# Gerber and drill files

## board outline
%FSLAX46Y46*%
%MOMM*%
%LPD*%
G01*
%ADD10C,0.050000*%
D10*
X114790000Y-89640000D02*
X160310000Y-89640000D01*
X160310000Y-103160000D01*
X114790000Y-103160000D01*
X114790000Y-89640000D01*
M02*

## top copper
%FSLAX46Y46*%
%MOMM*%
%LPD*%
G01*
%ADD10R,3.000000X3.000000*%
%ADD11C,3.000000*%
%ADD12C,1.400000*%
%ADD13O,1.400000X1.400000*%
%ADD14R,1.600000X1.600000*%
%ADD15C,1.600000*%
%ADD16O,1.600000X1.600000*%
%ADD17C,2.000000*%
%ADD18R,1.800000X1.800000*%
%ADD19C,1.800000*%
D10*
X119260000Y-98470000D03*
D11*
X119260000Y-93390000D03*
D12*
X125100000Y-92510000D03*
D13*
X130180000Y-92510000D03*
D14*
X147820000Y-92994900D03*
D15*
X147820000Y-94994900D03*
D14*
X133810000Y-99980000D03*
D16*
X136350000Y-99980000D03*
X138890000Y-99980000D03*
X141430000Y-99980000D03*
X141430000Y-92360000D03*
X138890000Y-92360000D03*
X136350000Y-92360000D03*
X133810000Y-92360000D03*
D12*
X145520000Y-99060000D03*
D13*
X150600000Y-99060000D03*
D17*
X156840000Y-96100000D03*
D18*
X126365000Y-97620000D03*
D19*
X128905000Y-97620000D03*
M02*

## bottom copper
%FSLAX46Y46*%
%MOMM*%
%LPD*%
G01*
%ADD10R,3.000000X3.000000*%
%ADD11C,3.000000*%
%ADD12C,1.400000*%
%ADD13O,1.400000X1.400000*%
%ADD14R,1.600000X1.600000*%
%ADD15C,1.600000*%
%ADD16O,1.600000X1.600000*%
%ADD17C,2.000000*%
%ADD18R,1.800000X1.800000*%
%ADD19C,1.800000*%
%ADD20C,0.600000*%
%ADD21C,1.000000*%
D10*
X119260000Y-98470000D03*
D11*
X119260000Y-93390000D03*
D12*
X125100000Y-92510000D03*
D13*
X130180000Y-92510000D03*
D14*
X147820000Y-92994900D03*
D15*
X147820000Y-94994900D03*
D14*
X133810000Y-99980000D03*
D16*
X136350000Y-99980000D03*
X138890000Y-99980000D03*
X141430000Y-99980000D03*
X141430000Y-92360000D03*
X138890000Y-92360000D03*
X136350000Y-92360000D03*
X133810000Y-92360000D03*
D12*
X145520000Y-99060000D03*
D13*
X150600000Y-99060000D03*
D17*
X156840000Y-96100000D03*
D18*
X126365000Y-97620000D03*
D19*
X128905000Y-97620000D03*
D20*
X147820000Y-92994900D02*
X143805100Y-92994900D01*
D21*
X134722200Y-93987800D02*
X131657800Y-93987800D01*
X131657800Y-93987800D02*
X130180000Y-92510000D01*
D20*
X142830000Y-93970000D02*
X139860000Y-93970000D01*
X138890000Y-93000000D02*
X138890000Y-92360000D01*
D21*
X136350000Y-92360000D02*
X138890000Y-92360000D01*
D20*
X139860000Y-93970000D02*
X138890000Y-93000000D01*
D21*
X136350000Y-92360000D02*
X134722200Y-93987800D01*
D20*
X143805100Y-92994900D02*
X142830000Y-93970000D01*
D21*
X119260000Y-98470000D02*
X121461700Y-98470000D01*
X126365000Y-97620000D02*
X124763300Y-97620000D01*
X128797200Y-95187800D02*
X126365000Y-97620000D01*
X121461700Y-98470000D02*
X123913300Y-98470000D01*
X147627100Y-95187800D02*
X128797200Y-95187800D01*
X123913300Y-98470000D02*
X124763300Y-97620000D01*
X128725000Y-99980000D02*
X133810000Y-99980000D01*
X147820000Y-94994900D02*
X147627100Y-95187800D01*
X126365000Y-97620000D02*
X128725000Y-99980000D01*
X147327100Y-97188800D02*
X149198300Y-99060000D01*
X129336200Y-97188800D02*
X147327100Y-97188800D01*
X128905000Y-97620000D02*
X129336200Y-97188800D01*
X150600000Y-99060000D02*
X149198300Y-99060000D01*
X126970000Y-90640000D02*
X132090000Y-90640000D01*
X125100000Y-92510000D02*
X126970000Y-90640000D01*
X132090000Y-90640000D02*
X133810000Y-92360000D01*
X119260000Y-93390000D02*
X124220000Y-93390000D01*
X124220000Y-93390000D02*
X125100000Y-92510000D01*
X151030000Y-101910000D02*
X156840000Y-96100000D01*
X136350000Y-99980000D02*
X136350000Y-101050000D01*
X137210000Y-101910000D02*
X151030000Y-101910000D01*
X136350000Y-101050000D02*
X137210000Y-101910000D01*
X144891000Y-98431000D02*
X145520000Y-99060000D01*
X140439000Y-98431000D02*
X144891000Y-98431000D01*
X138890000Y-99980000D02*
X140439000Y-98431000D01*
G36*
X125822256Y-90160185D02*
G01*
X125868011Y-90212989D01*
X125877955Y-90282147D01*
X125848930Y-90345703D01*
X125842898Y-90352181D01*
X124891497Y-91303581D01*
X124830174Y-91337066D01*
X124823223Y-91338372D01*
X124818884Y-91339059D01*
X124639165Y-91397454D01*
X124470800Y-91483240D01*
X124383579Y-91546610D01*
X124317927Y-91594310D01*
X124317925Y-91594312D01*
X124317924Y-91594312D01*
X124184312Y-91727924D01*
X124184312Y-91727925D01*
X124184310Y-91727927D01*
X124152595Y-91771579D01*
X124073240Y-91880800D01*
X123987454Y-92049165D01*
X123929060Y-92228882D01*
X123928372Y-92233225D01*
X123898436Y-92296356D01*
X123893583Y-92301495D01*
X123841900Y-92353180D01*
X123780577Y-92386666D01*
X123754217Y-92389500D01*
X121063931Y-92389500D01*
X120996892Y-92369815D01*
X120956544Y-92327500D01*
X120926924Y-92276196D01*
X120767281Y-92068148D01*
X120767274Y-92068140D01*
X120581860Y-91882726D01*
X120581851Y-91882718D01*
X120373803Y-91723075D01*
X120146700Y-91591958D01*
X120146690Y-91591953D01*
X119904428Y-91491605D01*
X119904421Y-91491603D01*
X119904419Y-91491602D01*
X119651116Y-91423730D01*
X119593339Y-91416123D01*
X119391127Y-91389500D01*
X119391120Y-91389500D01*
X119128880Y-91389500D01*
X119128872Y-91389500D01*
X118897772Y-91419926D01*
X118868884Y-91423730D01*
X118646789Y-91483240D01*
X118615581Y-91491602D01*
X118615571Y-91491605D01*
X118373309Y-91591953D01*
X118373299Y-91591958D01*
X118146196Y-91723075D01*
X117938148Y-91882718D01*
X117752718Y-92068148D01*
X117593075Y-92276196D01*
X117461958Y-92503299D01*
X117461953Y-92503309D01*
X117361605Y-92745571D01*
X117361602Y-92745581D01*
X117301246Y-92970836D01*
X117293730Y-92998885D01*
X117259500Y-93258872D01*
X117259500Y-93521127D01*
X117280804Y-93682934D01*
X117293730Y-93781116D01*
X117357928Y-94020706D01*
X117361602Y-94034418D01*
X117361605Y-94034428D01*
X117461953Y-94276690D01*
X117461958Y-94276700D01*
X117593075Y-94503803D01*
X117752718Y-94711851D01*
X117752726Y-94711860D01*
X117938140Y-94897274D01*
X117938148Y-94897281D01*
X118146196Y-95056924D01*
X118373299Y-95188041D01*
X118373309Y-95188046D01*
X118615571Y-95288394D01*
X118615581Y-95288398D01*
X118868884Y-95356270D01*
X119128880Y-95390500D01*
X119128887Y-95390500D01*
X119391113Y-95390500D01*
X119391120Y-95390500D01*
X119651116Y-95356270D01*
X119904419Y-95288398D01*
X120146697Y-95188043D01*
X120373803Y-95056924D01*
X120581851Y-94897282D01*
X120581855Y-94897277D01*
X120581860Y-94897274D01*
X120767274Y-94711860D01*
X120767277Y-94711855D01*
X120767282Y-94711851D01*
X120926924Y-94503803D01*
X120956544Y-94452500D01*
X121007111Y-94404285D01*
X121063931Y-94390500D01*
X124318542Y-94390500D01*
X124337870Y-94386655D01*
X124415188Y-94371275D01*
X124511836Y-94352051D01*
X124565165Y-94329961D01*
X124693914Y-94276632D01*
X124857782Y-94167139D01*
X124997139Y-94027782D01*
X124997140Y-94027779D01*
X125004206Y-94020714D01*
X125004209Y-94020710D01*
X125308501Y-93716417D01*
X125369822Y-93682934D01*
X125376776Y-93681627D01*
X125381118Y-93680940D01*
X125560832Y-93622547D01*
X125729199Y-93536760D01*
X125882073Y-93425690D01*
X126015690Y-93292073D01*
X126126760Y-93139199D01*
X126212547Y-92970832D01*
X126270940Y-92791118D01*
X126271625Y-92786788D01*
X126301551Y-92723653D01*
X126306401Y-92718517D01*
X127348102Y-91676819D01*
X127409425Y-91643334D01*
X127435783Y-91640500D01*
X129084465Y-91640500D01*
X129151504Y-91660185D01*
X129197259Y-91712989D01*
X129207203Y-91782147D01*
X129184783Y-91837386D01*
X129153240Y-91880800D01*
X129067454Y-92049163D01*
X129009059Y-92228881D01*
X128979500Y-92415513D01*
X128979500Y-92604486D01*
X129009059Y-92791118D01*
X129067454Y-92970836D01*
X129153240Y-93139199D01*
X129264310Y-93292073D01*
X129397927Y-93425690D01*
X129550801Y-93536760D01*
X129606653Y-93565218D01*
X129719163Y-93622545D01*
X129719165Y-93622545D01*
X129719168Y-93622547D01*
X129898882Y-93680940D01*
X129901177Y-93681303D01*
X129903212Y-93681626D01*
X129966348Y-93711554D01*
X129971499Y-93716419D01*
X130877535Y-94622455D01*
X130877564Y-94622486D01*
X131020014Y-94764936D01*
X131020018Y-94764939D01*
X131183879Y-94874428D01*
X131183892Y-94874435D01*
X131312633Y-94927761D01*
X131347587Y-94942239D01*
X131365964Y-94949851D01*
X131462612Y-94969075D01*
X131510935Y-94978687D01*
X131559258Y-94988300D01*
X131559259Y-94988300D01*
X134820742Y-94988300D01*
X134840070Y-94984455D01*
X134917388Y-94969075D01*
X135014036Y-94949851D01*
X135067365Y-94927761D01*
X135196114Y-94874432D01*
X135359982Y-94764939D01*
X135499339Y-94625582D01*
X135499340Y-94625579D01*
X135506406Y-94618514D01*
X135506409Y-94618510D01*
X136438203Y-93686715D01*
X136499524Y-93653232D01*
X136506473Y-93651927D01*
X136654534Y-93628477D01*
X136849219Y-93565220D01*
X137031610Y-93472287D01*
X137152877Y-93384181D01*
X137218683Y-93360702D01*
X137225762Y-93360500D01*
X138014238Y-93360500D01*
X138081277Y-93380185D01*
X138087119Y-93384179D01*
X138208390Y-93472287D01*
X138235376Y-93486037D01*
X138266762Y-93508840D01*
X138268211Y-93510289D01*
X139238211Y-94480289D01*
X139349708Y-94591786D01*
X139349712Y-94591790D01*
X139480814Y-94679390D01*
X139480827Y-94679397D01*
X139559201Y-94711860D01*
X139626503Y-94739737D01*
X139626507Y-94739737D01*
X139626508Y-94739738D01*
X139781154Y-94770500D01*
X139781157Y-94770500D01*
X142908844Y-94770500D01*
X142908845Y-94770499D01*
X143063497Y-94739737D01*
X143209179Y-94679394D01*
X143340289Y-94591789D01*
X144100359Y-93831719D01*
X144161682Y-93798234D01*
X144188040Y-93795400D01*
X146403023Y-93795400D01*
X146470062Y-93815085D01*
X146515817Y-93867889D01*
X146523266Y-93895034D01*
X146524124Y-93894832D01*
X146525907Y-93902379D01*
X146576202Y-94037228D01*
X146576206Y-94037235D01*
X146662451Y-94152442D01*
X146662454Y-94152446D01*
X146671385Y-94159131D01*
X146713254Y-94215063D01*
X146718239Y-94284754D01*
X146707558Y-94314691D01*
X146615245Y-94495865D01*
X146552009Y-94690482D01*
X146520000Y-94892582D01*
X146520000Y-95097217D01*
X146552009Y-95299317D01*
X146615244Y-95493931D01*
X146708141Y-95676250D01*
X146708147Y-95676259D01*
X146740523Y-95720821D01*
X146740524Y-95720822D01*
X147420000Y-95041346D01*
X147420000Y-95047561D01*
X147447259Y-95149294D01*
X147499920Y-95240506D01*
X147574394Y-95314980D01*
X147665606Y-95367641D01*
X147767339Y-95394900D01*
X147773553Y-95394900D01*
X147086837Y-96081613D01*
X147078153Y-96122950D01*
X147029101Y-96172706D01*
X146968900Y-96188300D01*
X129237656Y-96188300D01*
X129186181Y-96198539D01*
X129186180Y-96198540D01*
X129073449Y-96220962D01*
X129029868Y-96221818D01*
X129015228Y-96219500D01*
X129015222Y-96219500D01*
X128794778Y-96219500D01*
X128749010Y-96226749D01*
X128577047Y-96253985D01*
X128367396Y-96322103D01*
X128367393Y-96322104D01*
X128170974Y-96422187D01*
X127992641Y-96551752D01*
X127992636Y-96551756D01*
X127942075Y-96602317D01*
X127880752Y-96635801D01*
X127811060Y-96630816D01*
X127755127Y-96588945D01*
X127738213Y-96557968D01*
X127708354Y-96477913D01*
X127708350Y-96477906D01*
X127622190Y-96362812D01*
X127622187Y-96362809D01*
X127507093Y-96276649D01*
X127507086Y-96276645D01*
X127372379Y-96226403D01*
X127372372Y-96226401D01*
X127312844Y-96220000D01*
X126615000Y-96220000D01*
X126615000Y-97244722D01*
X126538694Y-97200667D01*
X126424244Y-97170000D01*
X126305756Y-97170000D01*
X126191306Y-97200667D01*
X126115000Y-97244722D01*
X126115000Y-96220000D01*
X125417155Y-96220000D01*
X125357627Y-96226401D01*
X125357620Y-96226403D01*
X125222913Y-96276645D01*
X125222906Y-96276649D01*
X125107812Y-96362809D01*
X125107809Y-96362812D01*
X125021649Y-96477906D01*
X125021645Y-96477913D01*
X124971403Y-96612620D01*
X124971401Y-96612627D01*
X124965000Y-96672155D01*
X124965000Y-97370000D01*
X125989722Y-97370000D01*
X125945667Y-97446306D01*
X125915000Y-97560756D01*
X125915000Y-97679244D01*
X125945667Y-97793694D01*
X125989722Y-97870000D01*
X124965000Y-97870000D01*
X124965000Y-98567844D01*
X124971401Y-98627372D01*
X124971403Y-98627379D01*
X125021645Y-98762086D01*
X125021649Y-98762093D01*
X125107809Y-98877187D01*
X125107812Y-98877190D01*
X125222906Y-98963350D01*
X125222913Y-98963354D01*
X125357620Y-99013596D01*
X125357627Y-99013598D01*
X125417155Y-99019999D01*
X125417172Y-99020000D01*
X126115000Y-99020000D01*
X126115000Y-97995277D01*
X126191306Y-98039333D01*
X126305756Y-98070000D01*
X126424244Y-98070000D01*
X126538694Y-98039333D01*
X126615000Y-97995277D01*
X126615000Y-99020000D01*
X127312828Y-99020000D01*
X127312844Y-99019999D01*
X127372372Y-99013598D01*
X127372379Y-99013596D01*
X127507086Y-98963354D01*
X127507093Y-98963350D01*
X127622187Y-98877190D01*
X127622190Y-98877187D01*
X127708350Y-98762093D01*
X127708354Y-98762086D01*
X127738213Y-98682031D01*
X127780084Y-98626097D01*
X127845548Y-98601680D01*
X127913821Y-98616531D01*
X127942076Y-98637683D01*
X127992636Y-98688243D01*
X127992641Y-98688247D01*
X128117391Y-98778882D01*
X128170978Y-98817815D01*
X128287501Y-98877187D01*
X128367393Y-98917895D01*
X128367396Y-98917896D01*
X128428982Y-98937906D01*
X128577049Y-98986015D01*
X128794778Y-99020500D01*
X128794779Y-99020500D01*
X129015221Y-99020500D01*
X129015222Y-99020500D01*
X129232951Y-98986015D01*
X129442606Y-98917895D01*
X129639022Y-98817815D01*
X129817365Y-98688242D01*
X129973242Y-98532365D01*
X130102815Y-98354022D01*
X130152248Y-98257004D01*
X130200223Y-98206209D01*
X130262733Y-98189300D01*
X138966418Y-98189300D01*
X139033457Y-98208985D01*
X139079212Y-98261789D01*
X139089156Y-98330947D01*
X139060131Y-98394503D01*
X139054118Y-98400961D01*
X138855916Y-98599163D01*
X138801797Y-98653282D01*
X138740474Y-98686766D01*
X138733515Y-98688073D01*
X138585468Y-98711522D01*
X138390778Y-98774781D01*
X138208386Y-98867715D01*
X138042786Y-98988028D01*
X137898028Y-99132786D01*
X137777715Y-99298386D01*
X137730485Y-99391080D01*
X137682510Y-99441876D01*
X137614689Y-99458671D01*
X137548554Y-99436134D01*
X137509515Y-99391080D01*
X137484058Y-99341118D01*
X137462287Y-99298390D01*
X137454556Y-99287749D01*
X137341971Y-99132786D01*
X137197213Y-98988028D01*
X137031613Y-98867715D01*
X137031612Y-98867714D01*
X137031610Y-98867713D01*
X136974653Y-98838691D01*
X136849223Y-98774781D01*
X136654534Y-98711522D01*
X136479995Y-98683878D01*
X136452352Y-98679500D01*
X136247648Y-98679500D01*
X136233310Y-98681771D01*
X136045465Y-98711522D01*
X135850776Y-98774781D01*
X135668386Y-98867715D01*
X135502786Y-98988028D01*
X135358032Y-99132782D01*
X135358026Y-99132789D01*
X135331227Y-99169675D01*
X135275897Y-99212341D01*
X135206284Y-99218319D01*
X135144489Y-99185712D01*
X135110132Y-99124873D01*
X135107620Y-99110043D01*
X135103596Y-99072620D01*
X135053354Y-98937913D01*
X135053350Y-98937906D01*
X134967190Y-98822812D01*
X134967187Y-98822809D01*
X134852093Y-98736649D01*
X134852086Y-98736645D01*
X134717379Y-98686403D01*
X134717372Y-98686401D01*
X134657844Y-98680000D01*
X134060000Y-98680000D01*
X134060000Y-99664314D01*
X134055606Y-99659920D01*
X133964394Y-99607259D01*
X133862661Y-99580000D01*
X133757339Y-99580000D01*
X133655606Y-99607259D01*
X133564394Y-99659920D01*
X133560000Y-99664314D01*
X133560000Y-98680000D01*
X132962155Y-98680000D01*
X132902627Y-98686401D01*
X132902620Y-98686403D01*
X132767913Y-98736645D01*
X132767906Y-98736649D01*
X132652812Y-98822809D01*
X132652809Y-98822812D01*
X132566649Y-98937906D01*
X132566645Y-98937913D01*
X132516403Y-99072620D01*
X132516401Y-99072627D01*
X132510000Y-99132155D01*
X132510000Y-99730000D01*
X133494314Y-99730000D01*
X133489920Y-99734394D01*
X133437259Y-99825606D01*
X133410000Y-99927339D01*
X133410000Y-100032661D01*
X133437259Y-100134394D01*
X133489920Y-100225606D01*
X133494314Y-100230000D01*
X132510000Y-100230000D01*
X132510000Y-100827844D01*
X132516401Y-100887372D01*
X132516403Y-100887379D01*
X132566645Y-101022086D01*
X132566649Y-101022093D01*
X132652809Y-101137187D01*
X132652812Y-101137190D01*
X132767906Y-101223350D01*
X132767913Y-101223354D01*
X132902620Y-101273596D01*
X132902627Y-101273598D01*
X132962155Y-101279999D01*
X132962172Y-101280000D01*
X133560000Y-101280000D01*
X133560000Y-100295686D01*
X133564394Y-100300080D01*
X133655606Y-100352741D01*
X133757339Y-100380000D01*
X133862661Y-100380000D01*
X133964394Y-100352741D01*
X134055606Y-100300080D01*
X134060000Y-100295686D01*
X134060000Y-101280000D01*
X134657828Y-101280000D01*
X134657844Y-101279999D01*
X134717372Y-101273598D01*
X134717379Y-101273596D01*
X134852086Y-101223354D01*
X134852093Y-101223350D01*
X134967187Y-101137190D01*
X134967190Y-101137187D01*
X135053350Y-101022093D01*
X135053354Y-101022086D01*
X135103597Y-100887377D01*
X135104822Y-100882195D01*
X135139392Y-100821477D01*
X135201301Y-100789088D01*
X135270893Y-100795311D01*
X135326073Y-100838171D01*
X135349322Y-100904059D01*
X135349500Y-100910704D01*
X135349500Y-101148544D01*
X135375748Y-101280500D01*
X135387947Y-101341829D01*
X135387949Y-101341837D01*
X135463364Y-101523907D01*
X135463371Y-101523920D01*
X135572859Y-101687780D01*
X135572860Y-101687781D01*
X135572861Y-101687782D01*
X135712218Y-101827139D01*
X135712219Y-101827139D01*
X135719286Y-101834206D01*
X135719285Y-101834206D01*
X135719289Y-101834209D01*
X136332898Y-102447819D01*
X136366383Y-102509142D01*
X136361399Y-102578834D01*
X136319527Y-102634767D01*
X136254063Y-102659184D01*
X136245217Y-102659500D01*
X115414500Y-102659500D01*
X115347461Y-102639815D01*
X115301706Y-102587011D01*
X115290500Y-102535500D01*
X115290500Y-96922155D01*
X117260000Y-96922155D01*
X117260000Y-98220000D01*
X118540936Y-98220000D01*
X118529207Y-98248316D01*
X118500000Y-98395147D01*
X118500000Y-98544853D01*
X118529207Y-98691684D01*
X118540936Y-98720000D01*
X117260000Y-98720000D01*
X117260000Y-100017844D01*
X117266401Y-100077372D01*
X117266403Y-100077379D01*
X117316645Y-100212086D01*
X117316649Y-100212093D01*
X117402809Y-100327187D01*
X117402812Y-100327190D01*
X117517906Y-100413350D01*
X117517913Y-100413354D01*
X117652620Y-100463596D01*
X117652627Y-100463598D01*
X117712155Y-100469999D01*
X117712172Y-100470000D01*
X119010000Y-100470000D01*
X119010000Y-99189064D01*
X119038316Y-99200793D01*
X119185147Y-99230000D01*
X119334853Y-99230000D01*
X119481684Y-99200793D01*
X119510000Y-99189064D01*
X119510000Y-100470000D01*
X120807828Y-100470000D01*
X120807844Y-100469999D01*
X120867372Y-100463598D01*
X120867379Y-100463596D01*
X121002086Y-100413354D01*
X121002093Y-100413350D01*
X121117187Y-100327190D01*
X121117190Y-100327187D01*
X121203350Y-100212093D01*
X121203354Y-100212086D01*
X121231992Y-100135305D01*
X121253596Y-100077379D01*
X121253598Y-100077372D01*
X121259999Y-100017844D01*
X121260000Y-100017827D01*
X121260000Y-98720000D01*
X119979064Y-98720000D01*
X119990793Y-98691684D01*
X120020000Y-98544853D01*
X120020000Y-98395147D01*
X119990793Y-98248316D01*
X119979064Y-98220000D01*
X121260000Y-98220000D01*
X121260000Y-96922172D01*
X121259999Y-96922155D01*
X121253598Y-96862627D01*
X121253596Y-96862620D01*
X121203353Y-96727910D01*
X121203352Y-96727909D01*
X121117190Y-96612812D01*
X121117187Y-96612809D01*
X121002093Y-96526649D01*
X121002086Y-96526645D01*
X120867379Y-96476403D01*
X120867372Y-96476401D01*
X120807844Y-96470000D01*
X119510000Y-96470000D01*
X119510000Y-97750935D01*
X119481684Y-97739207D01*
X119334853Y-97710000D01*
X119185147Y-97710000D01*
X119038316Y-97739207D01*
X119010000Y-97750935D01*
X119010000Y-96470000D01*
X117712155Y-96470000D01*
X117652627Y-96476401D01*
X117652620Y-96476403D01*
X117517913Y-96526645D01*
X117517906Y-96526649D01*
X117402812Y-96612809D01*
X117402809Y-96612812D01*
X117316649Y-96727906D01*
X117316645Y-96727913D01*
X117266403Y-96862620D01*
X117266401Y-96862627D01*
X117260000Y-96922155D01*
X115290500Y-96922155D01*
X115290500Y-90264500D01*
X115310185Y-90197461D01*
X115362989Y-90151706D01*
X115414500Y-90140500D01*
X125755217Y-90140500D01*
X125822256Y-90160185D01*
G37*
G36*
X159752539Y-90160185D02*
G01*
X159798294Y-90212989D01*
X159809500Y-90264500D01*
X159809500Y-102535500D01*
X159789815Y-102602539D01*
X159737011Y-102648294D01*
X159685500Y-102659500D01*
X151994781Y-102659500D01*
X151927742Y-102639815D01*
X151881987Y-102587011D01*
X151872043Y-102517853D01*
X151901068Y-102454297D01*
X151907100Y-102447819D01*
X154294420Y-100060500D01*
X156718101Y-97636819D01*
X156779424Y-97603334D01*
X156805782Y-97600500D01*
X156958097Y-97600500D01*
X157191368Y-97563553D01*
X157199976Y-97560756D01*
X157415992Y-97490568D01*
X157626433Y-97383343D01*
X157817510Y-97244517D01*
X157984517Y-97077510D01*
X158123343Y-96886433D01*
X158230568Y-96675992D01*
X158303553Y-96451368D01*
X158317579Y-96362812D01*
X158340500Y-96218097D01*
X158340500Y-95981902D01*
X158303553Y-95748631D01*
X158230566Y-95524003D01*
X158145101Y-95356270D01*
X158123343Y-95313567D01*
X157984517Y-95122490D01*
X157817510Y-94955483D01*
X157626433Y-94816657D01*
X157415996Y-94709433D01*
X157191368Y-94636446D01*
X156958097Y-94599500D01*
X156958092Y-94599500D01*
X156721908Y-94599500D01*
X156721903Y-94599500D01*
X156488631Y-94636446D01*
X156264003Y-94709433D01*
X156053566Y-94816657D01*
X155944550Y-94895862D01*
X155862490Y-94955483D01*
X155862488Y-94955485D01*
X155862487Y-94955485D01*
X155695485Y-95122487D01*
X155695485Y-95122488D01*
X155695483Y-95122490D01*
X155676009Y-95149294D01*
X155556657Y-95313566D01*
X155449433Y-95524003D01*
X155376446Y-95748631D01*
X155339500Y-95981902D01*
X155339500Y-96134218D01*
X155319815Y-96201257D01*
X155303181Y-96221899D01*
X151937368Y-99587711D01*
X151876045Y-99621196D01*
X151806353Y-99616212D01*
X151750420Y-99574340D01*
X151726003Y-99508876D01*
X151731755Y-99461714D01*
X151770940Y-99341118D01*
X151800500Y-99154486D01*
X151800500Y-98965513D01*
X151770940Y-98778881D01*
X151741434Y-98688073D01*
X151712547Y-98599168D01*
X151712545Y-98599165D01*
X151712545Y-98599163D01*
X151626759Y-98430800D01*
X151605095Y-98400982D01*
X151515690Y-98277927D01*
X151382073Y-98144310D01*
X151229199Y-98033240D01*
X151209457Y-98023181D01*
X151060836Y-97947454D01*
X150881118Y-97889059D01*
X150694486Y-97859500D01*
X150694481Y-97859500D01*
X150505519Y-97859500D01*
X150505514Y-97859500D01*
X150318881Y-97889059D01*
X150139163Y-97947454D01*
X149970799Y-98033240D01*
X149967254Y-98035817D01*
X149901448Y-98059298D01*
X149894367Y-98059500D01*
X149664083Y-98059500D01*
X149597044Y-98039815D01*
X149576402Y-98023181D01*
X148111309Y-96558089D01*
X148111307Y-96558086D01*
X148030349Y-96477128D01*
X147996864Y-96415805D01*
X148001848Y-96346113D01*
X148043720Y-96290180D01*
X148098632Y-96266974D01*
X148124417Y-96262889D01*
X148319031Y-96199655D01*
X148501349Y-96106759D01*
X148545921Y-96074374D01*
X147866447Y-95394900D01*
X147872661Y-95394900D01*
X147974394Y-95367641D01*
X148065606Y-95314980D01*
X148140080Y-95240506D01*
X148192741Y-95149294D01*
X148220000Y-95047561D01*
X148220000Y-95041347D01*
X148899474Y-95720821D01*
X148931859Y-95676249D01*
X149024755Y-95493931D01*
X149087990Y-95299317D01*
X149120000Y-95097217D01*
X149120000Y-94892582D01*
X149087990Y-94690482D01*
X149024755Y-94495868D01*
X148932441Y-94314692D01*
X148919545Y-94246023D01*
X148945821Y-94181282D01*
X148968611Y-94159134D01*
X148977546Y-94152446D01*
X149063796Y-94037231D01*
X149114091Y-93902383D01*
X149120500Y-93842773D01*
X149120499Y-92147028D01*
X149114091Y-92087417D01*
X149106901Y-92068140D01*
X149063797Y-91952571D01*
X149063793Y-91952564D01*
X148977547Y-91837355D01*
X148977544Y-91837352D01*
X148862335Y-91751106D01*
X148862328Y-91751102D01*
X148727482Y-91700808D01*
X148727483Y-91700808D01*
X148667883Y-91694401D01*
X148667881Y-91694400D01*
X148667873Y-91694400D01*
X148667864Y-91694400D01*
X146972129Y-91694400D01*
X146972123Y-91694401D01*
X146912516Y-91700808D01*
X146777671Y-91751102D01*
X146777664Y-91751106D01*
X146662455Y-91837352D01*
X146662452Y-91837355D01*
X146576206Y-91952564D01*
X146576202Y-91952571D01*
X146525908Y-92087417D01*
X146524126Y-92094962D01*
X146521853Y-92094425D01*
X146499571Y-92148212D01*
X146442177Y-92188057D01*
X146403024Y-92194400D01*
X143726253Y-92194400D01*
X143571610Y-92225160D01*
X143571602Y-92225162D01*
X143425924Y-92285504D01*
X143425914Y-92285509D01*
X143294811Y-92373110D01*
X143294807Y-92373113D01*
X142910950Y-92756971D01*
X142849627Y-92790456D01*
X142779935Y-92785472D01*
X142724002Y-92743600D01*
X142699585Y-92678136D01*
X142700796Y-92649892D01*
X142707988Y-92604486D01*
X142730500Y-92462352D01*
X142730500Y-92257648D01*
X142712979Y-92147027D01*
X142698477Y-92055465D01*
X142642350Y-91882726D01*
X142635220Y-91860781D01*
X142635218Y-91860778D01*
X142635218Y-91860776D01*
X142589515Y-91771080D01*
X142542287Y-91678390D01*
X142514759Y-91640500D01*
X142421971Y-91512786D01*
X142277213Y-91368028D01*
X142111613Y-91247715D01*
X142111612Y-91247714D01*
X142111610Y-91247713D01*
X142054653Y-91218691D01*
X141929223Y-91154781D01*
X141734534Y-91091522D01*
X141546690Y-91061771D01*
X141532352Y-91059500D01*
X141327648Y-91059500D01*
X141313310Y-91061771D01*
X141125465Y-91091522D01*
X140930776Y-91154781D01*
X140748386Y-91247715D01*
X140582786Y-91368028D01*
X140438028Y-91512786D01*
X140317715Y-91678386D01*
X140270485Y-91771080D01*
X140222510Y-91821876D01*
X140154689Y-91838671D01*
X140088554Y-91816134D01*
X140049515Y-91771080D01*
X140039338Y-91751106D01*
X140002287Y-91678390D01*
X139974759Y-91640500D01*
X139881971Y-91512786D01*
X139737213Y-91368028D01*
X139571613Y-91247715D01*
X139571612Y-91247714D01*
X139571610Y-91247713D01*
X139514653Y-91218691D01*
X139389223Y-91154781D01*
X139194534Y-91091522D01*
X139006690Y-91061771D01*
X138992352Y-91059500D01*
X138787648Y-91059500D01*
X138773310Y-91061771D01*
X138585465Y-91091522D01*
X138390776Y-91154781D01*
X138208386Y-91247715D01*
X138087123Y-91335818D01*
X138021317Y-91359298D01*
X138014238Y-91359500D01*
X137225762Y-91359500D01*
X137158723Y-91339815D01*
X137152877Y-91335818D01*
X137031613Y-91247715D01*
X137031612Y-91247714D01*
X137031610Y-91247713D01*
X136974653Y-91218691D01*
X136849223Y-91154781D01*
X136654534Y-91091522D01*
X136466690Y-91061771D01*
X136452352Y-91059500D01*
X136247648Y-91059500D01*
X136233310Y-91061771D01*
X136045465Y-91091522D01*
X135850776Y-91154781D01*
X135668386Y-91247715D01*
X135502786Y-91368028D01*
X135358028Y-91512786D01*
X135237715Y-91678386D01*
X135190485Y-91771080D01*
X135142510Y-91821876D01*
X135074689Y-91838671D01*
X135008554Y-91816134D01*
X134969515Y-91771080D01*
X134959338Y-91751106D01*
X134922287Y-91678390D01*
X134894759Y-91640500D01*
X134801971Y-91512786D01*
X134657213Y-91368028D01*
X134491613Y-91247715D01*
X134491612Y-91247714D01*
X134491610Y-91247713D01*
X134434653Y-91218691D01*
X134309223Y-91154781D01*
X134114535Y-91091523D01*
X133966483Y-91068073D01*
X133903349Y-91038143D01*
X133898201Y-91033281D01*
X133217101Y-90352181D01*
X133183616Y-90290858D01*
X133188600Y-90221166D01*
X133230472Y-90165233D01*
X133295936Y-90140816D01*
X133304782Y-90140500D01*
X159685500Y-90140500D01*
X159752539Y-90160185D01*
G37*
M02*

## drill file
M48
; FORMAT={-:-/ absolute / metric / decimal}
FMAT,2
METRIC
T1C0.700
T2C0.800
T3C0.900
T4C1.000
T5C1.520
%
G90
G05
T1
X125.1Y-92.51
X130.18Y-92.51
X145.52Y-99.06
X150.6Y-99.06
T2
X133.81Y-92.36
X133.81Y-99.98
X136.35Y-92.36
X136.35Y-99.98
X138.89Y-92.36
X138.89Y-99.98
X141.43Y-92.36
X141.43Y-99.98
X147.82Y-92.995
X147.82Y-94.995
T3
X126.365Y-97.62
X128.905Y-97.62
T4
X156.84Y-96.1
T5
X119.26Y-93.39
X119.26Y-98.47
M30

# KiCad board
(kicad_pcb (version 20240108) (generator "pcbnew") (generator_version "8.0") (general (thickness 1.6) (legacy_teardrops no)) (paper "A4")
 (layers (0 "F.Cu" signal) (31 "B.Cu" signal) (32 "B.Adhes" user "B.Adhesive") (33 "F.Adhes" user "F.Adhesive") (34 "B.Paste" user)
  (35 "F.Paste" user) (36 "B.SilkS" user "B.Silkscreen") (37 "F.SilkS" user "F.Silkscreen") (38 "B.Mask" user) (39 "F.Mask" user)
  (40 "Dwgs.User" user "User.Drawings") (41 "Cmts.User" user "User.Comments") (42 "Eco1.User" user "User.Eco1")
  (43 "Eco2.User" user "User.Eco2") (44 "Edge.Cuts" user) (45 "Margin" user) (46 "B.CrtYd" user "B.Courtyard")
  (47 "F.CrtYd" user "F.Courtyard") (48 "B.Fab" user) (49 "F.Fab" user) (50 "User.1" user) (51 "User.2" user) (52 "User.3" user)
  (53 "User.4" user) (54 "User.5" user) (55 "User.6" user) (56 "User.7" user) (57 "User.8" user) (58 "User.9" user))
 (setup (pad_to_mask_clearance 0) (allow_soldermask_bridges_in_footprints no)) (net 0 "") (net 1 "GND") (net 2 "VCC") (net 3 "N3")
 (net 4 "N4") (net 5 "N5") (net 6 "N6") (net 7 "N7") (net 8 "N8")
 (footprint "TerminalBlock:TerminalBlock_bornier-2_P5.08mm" (layer "F.Cu") (at 119.26 98.47 90)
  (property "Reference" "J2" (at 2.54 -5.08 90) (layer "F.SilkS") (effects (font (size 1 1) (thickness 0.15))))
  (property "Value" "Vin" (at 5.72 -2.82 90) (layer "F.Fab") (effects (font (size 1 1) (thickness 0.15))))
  (pad "1" thru_hole rect (at 0 0 90) (size 3 3) (drill 1.52) (layers "*.Cu" "*.Mask") (remove_unused_layers no) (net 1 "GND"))
  (pad "2" thru_hole circle (at 5.08 0 90) (size 3 3) (drill 1.52) (layers "*.Cu" "*.Mask") (remove_unused_layers no) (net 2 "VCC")))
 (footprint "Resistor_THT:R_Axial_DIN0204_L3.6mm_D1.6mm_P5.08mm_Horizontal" (layer "F.Cu") (at 125.1 92.51)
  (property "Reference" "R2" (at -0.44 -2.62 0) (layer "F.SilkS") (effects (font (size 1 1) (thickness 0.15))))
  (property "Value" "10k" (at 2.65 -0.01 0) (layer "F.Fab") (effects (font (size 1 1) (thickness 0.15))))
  (pad "1" thru_hole circle (at 0 0) (size 1.4 1.4) (drill 0.7) (layers "*.Cu" "*.Mask") (remove_unused_layers no) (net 2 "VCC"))
  (pad "2" thru_hole oval (at 5.08 0) (size 1.4 1.4) (drill 0.7) (layers "*.Cu" "*.Mask") (remove_unused_layers no) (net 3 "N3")))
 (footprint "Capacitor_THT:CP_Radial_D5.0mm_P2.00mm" (layer "F.Cu") (at 147.82 92.9949 -90)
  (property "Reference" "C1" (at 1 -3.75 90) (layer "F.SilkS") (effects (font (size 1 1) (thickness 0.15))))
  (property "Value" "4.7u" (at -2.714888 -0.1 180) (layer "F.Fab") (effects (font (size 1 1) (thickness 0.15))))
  (pad "1" thru_hole rect (at 0 0 270) (size 1.6 1.6) (drill 0.8) (layers "*.Cu" "*.Mask") (remove_unused_layers no) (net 3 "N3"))
  (pad "2" thru_hole circle (at 2 0 270) (size 1.6 1.6) (drill 0.8) (layers "*.Cu" "*.Mask") (remove_unused_layers no) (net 1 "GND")))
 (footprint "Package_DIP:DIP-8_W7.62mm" (layer "F.Cu") (at 133.81 99.98 90)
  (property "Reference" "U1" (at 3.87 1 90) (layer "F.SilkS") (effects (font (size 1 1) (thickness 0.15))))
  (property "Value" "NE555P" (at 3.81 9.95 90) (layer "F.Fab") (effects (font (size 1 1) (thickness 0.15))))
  (pad "1" thru_hole rect (at 0 0 90) (size 1.6 1.6) (drill 0.8) (layers "*.Cu" "*.Mask") (remove_unused_layers no) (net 1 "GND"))
  (pad "2" thru_hole oval (at 0 2.54 90) (size 1.6 1.6) (drill 0.8) (layers "*.Cu" "*.Mask") (remove_unused_layers no) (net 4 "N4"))
  (pad "3" thru_hole oval (at 0 5.08 90) (size 1.6 1.6) (drill 0.8) (layers "*.Cu" "*.Mask") (remove_unused_layers no) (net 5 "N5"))
  (pad "4" thru_hole oval (at 0 7.62 90) (size 1.6 1.6) (drill 0.8) (layers "*.Cu" "*.Mask") (remove_unused_layers no) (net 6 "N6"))
  (pad "5" thru_hole oval (at 7.62 7.62 90) (size 1.6 1.6) (drill 0.8) (layers "*.Cu" "*.Mask") (remove_unused_layers no) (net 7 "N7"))
  (pad "6" thru_hole oval (at 7.62 5.08 90) (size 1.6 1.6) (drill 0.8) (layers "*.Cu" "*.Mask") (remove_unused_layers no) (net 3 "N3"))
  (pad "7" thru_hole oval (at 7.62 2.54 90) (size 1.6 1.6) (drill 0.8) (layers "*.Cu" "*.Mask") (remove_unused_layers no) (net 3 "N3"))
  (pad "8" thru_hole oval (at 7.62 0 90) (size 1.6 1.6) (drill 0.8) (layers "*.Cu" "*.Mask") (remove_unused_layers no) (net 2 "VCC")))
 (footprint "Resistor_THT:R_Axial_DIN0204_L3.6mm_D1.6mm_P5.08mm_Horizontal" (layer "F.Cu") (at 145.52 99.06)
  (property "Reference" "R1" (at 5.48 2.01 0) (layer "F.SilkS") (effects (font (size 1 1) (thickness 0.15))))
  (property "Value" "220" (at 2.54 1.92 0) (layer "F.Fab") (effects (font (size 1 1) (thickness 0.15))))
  (pad "1" thru_hole circle (at 0 0) (size 1.4 1.4) (drill 0.7) (layers "*.Cu" "*.Mask") (remove_unused_layers no) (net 5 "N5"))
  (pad "2" thru_hole oval (at 5.08 0) (size 1.4 1.4) (drill 0.7) (layers "*.Cu" "*.Mask") (remove_unused_layers no) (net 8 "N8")))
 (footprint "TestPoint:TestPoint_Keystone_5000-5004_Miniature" (layer "F.Cu") (at 156.84 96.1)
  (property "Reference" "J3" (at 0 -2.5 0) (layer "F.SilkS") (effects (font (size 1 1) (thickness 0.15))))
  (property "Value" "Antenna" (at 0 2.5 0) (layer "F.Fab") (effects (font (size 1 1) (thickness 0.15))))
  (pad "1" thru_hole circle (at 0 0) (size 2 2) (drill 1) (layers "*.Cu" "*.Mask") (remove_unused_layers no) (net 4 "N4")))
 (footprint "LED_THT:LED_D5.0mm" (layer "F.Cu") (at 126.365 97.62)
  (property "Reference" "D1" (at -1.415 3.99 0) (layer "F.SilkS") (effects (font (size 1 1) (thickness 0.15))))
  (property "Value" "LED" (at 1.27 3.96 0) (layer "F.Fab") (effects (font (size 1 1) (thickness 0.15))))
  (pad "1" thru_hole rect (at 0 0) (size 1.8 1.8) (drill 0.9) (layers "*.Cu" "*.Mask") (remove_unused_layers no) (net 1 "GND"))
  (pad "2" thru_hole circle (at 2.54 0) (size 1.8 1.8) (drill 0.9) (layers "*.Cu" "*.Mask") (remove_unused_layers no) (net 8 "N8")))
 (gr_rect (start 114.79 89.64) (end 160.31 103.16) (stroke (width 0.05) (type default)) (fill none) (layer "Edge.Cuts"))
 (segment (start 147.82 92.9949) (end 143.8051 92.9949) (width 0.6) (layer "B.Cu") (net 3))
 (segment (start 134.7222 93.9878) (end 131.6578 93.9878) (width 1) (layer "B.Cu") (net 3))
 (segment (start 131.6578 93.9878) (end 130.18 92.51) (width 1) (layer "B.Cu") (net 3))
 (segment (start 142.83 93.97) (end 139.86 93.97) (width 0.6) (layer "B.Cu") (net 3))
 (segment (start 138.89 93) (end 138.89 92.36) (width 0.6) (layer "B.Cu") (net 3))
 (segment (start 136.35 92.36) (end 138.89 92.36) (width 1) (layer "B.Cu") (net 3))
 (segment (start 139.86 93.97) (end 138.89 93) (width 0.6) (layer "B.Cu") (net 3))
 (segment (start 136.35 92.36) (end 134.7222 93.9878) (width 1) (layer "B.Cu") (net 3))
 (segment (start 143.8051 92.9949) (end 142.83 93.97) (width 0.6) (layer "B.Cu") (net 3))
 (segment (start 119.26 98.47) (end 121.4617 98.47) (width 1) (layer "B.Cu") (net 1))
 (segment (start 126.365 97.62) (end 124.7633 97.62) (width 1) (layer "B.Cu") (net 1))
 (segment (start 128.7972 95.1878) (end 126.365 97.62) (width 1) (layer "B.Cu") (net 1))
 (segment (start 121.4617 98.47) (end 123.9133 98.47) (width 1) (layer "B.Cu") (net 1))
 (segment (start 147.6271 95.1878) (end 128.7972 95.1878) (width 1) (layer "B.Cu") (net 1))
 (segment (start 123.9133 98.47) (end 124.7633 97.62) (width 1) (layer "B.Cu") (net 1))
 (segment (start 128.725 99.98) (end 133.81 99.98) (width 1) (layer "B.Cu") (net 1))
 (segment (start 147.82 94.9949) (end 147.6271 95.1878) (width 1) (layer "B.Cu") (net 1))
 (segment (start 126.365 97.62) (end 128.725 99.98) (width 1) (layer "B.Cu") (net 1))
 (segment (start 147.3271 97.1888) (end 149.1983 99.06) (width 1) (layer "B.Cu") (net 8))
 (segment (start 129.3362 97.1888) (end 147.3271 97.1888) (width 1) (layer "B.Cu") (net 8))
 (segment (start 128.905 97.62) (end 129.3362 97.1888) (width 1) (layer "B.Cu") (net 8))
 (segment (start 150.6 99.06) (end 149.1983 99.06) (width 1) (layer "B.Cu") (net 8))
 (segment (start 126.97 90.64) (end 132.09 90.64) (width 1) (layer "B.Cu") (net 2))
 (segment (start 125.1 92.51) (end 126.97 90.64) (width 1) (layer "B.Cu") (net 2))
 (segment (start 132.09 90.64) (end 133.81 92.36) (width 1) (layer "B.Cu") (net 2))
 (segment (start 119.26 93.39) (end 124.22 93.39) (width 1) (layer "B.Cu") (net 2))
 (segment (start 124.22 93.39) (end 125.1 92.51) (width 1) (layer "B.Cu") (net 2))
 (segment (start 151.03 101.91) (end 156.84 96.1) (width 1) (layer "B.Cu") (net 4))
 (segment (start 136.35 99.98) (end 136.35 101.05) (width 1) (layer "B.Cu") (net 4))
 (segment (start 137.21 101.91) (end 151.03 101.91) (width 1) (layer "B.Cu") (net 4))
 (segment (start 136.35 101.05) (end 137.21 101.91) (width 1) (layer "B.Cu") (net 4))
 (segment (start 144.891 98.431) (end 145.52 99.06) (width 1) (layer "B.Cu") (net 5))
 (segment (start 140.439 98.431) (end 144.891 98.431) (width 1) (layer "B.Cu") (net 5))
 (segment (start 138.89 99.98) (end 140.439 98.431) (width 1) (layer "B.Cu") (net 5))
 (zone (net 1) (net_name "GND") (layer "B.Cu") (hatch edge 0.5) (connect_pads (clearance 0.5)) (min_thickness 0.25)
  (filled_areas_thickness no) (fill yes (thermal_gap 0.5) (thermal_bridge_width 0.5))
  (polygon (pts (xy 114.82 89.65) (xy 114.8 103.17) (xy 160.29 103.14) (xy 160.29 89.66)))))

